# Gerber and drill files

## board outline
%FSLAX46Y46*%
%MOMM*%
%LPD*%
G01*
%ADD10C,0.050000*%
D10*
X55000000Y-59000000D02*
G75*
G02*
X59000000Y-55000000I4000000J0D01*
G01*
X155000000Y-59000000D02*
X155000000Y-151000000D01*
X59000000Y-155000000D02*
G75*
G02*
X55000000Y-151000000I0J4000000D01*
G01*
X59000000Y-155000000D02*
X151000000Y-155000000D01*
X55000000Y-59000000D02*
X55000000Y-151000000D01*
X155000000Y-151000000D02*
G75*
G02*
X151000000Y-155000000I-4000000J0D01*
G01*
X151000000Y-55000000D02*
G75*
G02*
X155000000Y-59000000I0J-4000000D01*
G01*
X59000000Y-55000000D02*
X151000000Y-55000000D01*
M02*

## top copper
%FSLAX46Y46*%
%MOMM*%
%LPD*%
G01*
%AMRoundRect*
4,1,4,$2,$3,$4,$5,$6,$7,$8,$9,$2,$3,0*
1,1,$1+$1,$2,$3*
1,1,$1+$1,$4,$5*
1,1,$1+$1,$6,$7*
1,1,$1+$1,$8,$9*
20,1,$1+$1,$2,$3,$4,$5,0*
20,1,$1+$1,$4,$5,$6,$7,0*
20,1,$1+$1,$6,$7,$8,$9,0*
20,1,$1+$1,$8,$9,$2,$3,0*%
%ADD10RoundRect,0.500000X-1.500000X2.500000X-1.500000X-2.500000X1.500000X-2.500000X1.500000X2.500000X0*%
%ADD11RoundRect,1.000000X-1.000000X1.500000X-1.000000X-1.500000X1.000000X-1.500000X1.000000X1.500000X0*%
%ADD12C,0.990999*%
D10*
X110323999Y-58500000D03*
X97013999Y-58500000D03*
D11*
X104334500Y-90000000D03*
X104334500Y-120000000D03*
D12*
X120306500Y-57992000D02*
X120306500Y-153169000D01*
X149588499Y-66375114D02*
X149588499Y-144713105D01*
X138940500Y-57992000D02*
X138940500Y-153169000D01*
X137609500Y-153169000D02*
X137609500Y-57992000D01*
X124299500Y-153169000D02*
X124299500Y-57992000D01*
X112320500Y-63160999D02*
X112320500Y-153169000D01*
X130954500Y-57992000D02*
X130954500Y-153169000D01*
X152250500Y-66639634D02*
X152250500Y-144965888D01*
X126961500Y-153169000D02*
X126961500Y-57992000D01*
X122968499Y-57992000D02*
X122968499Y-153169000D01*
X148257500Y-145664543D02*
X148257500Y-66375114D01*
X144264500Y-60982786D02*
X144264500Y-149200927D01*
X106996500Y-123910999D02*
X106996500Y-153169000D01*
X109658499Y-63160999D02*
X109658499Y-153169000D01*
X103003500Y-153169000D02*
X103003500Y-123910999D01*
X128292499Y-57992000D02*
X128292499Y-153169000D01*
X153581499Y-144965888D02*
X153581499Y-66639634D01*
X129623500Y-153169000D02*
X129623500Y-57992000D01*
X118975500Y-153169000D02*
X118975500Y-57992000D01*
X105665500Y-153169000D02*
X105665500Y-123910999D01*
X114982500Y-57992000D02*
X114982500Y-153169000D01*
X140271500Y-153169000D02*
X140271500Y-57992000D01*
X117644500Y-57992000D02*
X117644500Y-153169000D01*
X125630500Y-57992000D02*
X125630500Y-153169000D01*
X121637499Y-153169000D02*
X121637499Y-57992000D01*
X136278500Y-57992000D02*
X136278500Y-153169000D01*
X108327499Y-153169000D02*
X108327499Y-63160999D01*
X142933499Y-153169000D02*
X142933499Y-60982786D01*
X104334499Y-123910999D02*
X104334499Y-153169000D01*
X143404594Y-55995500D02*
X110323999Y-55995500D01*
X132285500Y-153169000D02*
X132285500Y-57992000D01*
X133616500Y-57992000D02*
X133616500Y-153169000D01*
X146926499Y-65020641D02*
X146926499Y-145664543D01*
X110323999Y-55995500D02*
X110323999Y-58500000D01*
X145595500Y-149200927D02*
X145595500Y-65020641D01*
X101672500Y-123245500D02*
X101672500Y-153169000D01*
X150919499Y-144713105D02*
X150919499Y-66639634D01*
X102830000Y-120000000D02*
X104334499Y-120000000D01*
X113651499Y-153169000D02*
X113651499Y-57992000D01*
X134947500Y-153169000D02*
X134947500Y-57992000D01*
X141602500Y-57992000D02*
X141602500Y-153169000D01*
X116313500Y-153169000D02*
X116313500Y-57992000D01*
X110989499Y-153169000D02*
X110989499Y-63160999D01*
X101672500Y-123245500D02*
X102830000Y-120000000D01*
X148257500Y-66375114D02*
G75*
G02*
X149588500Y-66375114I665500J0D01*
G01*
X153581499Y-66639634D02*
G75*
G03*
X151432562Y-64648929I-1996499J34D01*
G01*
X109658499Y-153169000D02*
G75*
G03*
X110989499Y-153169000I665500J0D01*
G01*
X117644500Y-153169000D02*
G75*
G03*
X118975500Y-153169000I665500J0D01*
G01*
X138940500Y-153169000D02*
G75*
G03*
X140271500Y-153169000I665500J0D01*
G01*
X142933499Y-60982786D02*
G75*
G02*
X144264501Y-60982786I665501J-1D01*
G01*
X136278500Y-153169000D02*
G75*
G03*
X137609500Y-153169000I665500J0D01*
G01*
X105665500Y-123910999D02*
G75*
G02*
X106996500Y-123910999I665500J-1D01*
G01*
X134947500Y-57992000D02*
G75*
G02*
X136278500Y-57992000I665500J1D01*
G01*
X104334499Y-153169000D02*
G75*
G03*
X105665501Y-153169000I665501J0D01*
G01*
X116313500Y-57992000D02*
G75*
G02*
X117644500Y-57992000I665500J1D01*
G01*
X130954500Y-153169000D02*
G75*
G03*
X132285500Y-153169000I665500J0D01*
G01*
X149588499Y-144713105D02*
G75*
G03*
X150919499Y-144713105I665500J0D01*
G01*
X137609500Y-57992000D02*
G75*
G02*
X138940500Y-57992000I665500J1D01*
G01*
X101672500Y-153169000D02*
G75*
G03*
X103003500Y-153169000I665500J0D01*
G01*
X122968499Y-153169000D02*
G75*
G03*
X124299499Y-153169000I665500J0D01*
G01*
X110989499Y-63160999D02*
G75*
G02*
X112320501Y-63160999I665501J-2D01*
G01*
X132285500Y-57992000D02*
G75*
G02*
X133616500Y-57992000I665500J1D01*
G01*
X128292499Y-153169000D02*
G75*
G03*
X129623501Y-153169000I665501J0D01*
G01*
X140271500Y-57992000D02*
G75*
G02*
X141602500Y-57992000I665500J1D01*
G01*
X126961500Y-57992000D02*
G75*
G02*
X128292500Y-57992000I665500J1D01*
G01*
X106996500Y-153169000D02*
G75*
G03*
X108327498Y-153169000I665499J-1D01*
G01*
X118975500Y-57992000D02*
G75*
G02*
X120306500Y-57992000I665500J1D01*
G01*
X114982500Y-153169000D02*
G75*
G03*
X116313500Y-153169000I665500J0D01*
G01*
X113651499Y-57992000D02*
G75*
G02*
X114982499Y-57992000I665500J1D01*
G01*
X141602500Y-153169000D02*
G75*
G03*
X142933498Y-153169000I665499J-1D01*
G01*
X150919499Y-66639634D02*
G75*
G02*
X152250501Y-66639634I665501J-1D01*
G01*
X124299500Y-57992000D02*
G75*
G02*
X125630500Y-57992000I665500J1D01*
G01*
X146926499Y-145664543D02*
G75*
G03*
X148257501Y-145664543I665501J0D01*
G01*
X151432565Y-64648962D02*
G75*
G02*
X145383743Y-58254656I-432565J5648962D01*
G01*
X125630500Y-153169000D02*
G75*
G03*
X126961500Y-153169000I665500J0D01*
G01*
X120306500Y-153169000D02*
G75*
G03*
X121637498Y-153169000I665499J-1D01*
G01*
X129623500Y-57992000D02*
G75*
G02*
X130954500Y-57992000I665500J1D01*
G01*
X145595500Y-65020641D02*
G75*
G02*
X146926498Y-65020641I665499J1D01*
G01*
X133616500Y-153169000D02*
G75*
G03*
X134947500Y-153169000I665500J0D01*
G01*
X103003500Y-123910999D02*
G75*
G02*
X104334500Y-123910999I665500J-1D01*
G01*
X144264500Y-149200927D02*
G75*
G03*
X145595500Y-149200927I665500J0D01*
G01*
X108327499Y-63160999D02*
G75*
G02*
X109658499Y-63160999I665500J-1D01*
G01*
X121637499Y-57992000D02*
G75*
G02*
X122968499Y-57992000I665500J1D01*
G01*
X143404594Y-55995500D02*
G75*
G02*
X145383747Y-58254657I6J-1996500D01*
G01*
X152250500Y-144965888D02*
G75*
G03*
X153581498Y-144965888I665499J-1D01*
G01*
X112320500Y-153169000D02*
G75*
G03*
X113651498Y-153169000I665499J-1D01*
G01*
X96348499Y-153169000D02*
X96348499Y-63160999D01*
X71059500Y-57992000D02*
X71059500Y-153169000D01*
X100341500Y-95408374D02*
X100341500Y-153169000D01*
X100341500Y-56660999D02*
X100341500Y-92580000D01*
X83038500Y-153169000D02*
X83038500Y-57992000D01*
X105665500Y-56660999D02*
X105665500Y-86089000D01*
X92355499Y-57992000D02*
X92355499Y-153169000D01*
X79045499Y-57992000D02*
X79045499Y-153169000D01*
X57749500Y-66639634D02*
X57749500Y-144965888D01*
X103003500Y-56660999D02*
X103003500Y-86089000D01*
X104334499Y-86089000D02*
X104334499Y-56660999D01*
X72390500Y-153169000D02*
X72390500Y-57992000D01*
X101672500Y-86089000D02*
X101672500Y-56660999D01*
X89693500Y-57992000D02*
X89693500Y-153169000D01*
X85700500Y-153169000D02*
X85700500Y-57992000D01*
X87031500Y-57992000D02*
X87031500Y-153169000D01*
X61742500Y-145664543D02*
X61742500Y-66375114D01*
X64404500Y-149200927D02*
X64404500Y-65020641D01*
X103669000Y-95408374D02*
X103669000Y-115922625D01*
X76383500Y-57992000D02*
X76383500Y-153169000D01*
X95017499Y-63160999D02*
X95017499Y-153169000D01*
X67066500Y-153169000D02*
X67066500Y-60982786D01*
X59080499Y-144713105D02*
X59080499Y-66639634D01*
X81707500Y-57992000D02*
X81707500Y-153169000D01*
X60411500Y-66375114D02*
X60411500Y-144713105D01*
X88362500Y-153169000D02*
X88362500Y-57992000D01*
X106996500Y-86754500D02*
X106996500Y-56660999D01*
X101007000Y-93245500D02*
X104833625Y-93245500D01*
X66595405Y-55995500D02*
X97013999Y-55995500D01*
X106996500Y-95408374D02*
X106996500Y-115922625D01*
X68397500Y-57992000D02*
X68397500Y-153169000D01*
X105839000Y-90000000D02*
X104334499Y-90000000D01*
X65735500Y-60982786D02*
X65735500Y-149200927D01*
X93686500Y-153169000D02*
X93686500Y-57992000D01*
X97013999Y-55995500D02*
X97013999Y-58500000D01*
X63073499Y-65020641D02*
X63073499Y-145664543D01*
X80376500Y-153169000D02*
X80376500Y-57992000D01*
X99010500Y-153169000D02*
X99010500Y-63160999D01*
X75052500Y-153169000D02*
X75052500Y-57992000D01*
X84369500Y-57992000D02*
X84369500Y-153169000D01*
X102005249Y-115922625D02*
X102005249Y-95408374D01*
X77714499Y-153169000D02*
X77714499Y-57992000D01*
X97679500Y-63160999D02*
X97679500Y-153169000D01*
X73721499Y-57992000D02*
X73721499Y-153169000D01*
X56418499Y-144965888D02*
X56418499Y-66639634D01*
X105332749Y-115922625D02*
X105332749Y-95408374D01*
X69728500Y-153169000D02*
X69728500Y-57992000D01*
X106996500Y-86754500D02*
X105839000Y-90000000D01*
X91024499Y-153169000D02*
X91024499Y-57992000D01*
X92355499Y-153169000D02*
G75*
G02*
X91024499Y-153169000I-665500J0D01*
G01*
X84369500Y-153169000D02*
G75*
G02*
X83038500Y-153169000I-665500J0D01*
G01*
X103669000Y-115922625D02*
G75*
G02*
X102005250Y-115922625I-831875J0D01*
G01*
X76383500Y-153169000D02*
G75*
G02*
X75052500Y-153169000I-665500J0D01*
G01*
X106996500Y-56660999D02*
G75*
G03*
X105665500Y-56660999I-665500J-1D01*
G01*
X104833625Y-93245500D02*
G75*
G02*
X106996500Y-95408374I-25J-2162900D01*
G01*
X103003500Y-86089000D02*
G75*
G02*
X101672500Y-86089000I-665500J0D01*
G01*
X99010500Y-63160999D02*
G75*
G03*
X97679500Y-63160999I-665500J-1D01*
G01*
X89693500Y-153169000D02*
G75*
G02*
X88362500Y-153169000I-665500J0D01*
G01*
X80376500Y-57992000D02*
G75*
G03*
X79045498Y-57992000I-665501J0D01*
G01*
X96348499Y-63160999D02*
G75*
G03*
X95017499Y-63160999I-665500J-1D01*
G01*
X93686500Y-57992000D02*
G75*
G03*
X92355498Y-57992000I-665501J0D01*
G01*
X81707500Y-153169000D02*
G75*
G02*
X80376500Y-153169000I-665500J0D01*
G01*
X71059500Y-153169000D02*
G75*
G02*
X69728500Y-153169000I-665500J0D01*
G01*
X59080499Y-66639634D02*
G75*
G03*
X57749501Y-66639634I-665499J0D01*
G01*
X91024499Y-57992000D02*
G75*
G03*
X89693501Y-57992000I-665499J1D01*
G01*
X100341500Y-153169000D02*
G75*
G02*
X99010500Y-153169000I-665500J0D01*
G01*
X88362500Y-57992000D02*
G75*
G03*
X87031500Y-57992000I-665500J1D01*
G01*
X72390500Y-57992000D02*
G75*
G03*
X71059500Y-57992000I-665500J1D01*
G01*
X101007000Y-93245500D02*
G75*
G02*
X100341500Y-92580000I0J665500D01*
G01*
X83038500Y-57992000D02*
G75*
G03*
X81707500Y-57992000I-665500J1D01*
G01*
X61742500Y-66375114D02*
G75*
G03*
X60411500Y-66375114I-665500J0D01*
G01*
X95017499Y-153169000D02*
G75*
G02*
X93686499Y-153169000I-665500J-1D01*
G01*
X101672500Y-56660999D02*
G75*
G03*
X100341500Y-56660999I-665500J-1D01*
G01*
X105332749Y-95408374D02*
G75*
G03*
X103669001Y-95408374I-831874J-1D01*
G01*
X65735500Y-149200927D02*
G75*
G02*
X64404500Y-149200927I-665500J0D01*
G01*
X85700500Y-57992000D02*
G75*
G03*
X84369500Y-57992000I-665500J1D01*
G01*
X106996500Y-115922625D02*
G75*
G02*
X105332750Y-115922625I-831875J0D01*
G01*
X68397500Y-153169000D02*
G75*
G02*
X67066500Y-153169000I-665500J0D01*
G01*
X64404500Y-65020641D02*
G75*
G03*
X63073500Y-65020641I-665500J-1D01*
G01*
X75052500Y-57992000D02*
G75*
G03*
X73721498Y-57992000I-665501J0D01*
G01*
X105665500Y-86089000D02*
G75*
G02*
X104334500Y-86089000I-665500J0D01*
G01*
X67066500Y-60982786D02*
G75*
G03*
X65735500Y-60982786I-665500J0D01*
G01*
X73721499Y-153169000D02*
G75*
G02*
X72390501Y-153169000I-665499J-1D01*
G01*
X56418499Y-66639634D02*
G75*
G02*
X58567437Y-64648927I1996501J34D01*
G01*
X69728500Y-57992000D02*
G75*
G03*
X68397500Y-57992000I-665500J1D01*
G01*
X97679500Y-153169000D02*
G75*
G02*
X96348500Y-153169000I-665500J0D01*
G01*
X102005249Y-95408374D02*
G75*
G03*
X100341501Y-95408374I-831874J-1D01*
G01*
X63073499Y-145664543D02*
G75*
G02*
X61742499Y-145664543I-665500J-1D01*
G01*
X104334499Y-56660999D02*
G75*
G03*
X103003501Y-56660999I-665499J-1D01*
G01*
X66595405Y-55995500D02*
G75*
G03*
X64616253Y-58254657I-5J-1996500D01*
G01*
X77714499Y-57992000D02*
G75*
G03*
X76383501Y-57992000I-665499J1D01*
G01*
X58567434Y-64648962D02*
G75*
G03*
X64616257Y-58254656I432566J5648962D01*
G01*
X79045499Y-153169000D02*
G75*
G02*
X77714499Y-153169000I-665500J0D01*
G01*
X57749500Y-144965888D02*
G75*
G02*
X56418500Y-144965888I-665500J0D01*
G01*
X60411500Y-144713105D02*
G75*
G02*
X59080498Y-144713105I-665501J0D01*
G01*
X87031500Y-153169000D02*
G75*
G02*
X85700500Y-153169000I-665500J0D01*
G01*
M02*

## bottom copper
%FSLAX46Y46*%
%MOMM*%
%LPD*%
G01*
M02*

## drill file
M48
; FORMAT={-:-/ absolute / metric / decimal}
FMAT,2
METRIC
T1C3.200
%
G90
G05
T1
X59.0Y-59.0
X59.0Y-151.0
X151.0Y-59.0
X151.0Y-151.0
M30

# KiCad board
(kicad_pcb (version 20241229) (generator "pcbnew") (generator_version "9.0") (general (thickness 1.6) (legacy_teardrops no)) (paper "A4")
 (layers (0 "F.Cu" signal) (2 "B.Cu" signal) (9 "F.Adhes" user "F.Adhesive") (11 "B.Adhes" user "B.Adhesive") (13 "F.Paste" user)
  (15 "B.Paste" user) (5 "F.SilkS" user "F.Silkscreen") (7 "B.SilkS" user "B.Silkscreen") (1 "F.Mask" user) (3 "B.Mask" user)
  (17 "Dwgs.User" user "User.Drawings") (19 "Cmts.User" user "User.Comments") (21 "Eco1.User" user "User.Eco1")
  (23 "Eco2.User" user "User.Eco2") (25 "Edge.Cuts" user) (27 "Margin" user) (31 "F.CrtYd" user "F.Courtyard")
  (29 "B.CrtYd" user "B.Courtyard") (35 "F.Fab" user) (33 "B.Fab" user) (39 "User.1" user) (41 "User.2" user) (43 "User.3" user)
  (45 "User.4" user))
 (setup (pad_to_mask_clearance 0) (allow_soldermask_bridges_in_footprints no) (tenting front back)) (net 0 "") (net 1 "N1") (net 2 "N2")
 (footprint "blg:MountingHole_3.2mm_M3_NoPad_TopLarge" (layer "F.Cu") (at 151 59)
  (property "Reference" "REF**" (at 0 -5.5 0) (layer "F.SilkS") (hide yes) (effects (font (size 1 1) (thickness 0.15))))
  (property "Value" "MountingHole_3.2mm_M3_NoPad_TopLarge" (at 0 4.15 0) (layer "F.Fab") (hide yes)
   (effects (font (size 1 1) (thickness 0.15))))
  (pad "" np_thru_hole circle (at 0 0) (size 7.6 7.6) (drill 3.2) (layers) (zone_connect 2)))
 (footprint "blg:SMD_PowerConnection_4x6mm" (layer "F.Cu") (at 110.323999 58.5 -90)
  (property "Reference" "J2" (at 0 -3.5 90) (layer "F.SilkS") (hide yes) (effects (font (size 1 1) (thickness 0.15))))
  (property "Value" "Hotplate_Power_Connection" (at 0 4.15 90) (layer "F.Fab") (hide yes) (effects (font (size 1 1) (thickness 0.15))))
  (pad "1" smd roundrect (at 0 0 270) (size 6 4) (layers "F.Cu" "F.Mask" "F.Paste") (roundrect_rratio 0.125) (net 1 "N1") (zone_connect 2)))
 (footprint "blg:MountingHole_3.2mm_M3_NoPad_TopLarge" (layer "F.Cu") (at 59 151)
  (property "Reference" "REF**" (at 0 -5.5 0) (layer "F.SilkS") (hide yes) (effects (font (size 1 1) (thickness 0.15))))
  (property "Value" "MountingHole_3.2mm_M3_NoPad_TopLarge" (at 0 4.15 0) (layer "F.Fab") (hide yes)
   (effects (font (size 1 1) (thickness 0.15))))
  (pad "" np_thru_hole circle (at 0 0) (size 7.6 7.6) (drill 3.2) (layers) (zone_connect 2)))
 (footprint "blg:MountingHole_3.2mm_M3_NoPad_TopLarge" (layer "F.Cu") (at 151 151)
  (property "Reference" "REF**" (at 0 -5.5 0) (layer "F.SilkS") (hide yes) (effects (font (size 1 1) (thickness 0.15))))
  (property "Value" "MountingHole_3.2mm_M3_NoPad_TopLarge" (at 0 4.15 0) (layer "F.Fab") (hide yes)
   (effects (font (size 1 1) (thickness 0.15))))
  (pad "" np_thru_hole circle (at 0 0) (size 7.6 7.6) (drill 3.2) (layers) (zone_connect 2)))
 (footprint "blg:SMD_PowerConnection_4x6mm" (layer "F.Cu") (at 97.013999 58.5 -90)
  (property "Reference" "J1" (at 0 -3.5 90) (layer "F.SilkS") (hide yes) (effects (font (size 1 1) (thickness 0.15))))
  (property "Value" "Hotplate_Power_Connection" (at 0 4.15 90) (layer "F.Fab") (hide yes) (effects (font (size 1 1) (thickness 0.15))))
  (pad "1" smd roundrect (at 0 0 270) (size 6 4) (layers "F.Cu" "F.Mask" "F.Paste") (roundrect_rratio 0.125) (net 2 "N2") (zone_connect 2)))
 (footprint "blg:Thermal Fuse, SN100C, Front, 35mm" (layer "F.Cu") (at 104.3345 105 -90)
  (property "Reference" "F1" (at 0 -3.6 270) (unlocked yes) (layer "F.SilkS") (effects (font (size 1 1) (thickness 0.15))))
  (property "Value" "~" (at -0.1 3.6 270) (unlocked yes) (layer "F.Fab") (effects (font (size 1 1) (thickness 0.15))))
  (pad "1" smd roundrect (at -15 0 270) (size 5 4) (layers "F.Cu" "F.Mask") (roundrect_rratio 0.25) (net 2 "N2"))
  (pad "2" smd roundrect (at 15 0 270) (size 5 4) (layers "F.Cu" "F.Mask") (roundrect_rratio 0.25) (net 1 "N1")))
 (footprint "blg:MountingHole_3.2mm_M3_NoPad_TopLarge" (layer "F.Cu") (at 59 59)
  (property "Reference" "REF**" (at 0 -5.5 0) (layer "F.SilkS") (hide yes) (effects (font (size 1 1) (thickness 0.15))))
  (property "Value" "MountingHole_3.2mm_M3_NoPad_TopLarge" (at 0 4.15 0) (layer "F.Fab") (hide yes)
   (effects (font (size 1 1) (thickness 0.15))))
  (pad "" np_thru_hole circle (at 0 0) (size 7.6 7.6) (drill 3.2) (layers) (zone_connect 2)))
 (gr_arc (start 55 59) (mid 56.171573 56.171573) (end 59 55) (stroke (width 0.05) (type solid)) (layer "Edge.Cuts"))
 (gr_line (start 155 59) (end 155 151) (stroke (width 0.05) (type default)) (layer "Edge.Cuts"))
 (gr_arc (start 59 155) (mid 56.171573 153.828427) (end 55 151) (stroke (width 0.05) (type solid)) (layer "Edge.Cuts"))
 (gr_line (start 59 155) (end 151 155) (stroke (width 0.05) (type default)) (layer "Edge.Cuts"))
 (gr_line (start 55 59) (end 55 151) (stroke (width 0.05) (type default)) (layer "Edge.Cuts"))
 (gr_arc (start 155 151) (mid 153.828427 153.828427) (end 151 155) (stroke (width 0.05) (type solid)) (layer "Edge.Cuts"))
 (gr_arc (start 151 55) (mid 153.828427 56.171573) (end 155 59) (stroke (width 0.05) (type solid)) (layer "Edge.Cuts"))
 (gr_line (start 59 55) (end 151 55) (stroke (width 0.05) (type default)) (layer "Edge.Cuts"))
 (segment (start 120.3065 57.992) (end 120.3065 153.169) (width 0.990999) (layer "F.Cu") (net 1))
 (segment (start 149.588499 66.375114) (end 149.588499 144.713105) (width 0.990999) (layer "F.Cu") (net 1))
 (segment (start 138.9405 57.992) (end 138.9405 153.169) (width 0.990999) (layer "F.Cu") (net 1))
 (segment (start 137.6095 153.169) (end 137.6095 57.992) (width 0.990999) (layer "F.Cu") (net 1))
 (segment (start 124.2995 153.169) (end 124.2995 57.992) (width 0.990999) (layer "F.Cu") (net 1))
 (segment (start 112.3205 63.160999) (end 112.3205 153.169) (width 0.990999) (layer "F.Cu") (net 1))
 (segment (start 130.9545 57.992) (end 130.9545 153.169) (width 0.990999) (layer "F.Cu") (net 1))
 (segment (start 152.2505 66.639634) (end 152.2505 144.965888) (width 0.990999) (layer "F.Cu") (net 1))
 (segment (start 126.9615 153.169) (end 126.9615 57.992) (width 0.990999) (layer "F.Cu") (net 1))
 (segment (start 122.968499 57.992) (end 122.968499 153.169) (width 0.990999) (layer "F.Cu") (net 1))
 (segment (start 148.2575 145.664543) (end 148.2575 66.375114) (width 0.990999) (layer "F.Cu") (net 1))
 (segment (start 144.2645 60.982786) (end 144.2645 149.200927) (width 0.990999) (layer "F.Cu") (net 1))
 (segment (start 106.9965 123.910999) (end 106.9965 153.169) (width 0.990999) (layer "F.Cu") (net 1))
 (segment (start 109.658499 63.160999) (end 109.658499 153.169) (width 0.990999) (layer "F.Cu") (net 1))
 (segment (start 103.0035 153.169) (end 103.0035 123.910999) (width 0.990999) (layer "F.Cu") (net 1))
 (segment (start 128.292499 57.992) (end 128.292499 153.169) (width 0.990999) (layer "F.Cu") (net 1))
 (segment (start 153.581499 144.965888) (end 153.581499 66.639634) (width 0.990999) (layer "F.Cu") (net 1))
 (segment (start 129.6235 153.169) (end 129.6235 57.992) (width 0.990999) (layer "F.Cu") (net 1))
 (segment (start 118.9755 153.169) (end 118.9755 57.992) (width 0.990999) (layer "F.Cu") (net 1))
 (segment (start 105.6655 153.169) (end 105.6655 123.910999) (width 0.990999) (layer "F.Cu") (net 1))
 (segment (start 114.9825 57.992) (end 114.9825 153.169) (width 0.990999) (layer "F.Cu") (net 1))
 (segment (start 140.2715 153.169) (end 140.2715 57.992) (width 0.990999) (layer "F.Cu") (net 1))
 (segment (start 117.6445 57.992) (end 117.6445 153.169) (width 0.990999) (layer "F.Cu") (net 1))
 (segment (start 125.6305 57.992) (end 125.6305 153.169) (width 0.990999) (layer "F.Cu") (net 1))
 (segment (start 121.637499 153.169) (end 121.637499 57.992) (width 0.990999) (layer "F.Cu") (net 1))
 (segment (start 136.2785 57.992) (end 136.2785 153.169) (width 0.990999) (layer "F.Cu") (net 1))
 (segment (start 108.327499 153.169) (end 108.327499 63.160999) (width 0.990999) (layer "F.Cu") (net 1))
 (segment (start 142.933499 153.169) (end 142.933499 60.982786) (width 0.990999) (layer "F.Cu") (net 1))
 (segment (start 104.334499 123.910999) (end 104.334499 153.169) (width 0.990999) (layer "F.Cu") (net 1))
 (segment (start 143.404594 55.9955) (end 110.323999 55.9955) (width 0.990999) (layer "F.Cu") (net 1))
 (segment (start 132.2855 153.169) (end 132.2855 57.992) (width 0.990999) (layer "F.Cu") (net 1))
 (segment (start 133.6165 57.992) (end 133.6165 153.169) (width 0.990999) (layer "F.Cu") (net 1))
 (segment (start 146.926499 65.020641) (end 146.926499 145.664543) (width 0.990999) (layer "F.Cu") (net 1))
 (segment (start 110.323999 55.9955) (end 110.323999 58.5) (width 0.990999) (layer "F.Cu") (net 1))
 (segment (start 145.5955 149.200927) (end 145.5955 65.020641) (width 0.990999) (layer "F.Cu") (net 1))
 (segment (start 101.6725 123.2455) (end 101.6725 153.169) (width 0.990999) (layer "F.Cu") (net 1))
 (segment (start 150.919499 144.713105) (end 150.919499 66.639634) (width 0.990999) (layer "F.Cu") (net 1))
 (segment (start 102.83 120) (end 104.334499 120) (width 0.990999) (layer "F.Cu") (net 1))
 (segment (start 113.651499 153.169) (end 113.651499 57.992) (width 0.990999) (layer "F.Cu") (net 1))
 (segment (start 134.9475 153.169) (end 134.9475 57.992) (width 0.990999) (layer "F.Cu") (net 1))
 (segment (start 141.6025 57.992) (end 141.6025 153.169) (width 0.990999) (layer "F.Cu") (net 1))
 (segment (start 116.3135 153.169) (end 116.3135 57.992) (width 0.990999) (layer "F.Cu") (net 1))
 (segment (start 110.989499 153.169) (end 110.989499 63.160999) (width 0.990999) (layer "F.Cu") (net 1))
 (segment (start 101.6725 123.2455) (end 102.83 120) (width 0.990999) (layer "F.Cu") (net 1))
 (arc (start 148.2575 66.375114) (mid 148.923 65.709614) (end 149.588499 66.375114) (width 0.990999) (layer "F.Cu") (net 1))
 (arc (start 153.581499 66.639634) (mid 153.048645 65.281785) (end 151.432565 64.648962) (width 0.990999) (layer "F.Cu") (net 1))
 (arc (start 109.658499 153.169) (mid 110.324 153.8345) (end 110.989499 153.169) (width 0.990999) (layer "F.Cu") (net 1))
 (arc (start 117.6445 153.169) (mid 118.31 153.8345) (end 118.9755 153.169) (width 0.990999) (layer "F.Cu") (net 1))
 (arc (start 138.9405 153.169) (mid 139.605999 153.8345) (end 140.2715 153.169) (width 0.990999) (layer "F.Cu") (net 1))
 (arc (start 142.933499 60.982786) (mid 143.599 60.317286) (end 144.2645 60.982786) (width 0.990999) (layer "F.Cu") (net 1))
 (arc (start 136.2785 153.169) (mid 136.944 153.8345) (end 137.6095 153.169) (width 0.990999) (layer "F.Cu") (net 1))
 (arc (start 105.6655 123.910999) (mid 106.330999 123.2455) (end 106.9965 123.910999) (width 0.990999) (layer "F.Cu") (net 1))
 (arc (start 134.9475 57.992) (mid 135.612999 57.326499) (end 136.2785 57.992) (width 0.990999) (layer "F.Cu") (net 1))
 (arc (start 104.334499 153.169) (mid 105 153.8345) (end 105.6655 153.169) (width 0.990999) (layer "F.Cu") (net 1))
 (arc (start 116.3135 57.992) (mid 116.979 57.326499) (end 117.6445 57.992) (width 0.990999) (layer "F.Cu") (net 1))
 (arc (start 130.9545 153.169) (mid 131.619999 153.8345) (end 132.2855 153.169) (width 0.990999) (layer "F.Cu") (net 1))
 (arc (start 149.588499 144.713105) (mid 150.254 145.378605) (end 150.919499 144.713105) (width 0.990999) (layer "F.Cu") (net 1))
 (arc (start 137.6095 57.992) (mid 138.274999 57.326499) (end 138.9405 57.992) (width 0.990999) (layer "F.Cu") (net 1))
 (arc (start 101.6725 153.169) (mid 102.338 153.8345) (end 103.0035 153.169) (width 0.990999) (layer "F.Cu") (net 1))
 (arc (start 122.968499 153.169) (mid 123.634 153.8345) (end 124.2995 153.169) (width 0.990999) (layer "F.Cu") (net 1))
 (arc (start 110.989499 63.160999) (mid 111.654999 62.4955) (end 112.3205 63.160999) (width 0.990999) (layer "F.Cu") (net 1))
 (arc (start 132.2855 57.992) (mid 132.951 57.326499) (end 133.6165 57.992) (width 0.990999) (layer "F.Cu") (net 1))
 (arc (start 128.292499 153.169) (mid 128.958 153.8345) (end 129.6235 153.169) (width 0.990999) (layer "F.Cu") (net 1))
 (arc (start 140.2715 57.992) (mid 140.937 57.326499) (end 141.6025 57.992) (width 0.990999) (layer "F.Cu") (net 1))
 (arc (start 126.9615 57.992) (mid 127.627 57.326499) (end 128.292499 57.992) (width 0.990999) (layer "F.Cu") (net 1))
 (arc (start 106.9965 153.169) (mid 107.661999 153.8345) (end 108.327499 153.169) (width 0.990999) (layer "F.Cu") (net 1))
 (arc (start 118.9755 57.992) (mid 119.640999 57.326499) (end 120.3065 57.992) (width 0.990999) (layer "F.Cu") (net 1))
 (arc (start 114.9825 153.169) (mid 115.648 153.8345) (end 116.3135 153.169) (width 0.990999) (layer "F.Cu") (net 1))
 (arc (start 113.651499 57.992) (mid 114.317 57.326499) (end 114.9825 57.992) (width 0.990999) (layer "F.Cu") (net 1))
 (arc (start 141.6025 153.169) (mid 142.268 153.8345) (end 142.933499 153.169) (width 0.990999) (layer "F.Cu") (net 1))
 (arc (start 150.919499 66.639634) (mid 151.585 65.974134) (end 152.2505 66.639634) (width 0.990999) (layer "F.Cu") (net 1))
 (arc (start 124.2995 57.992) (mid 124.964999 57.326499) (end 125.6305 57.992) (width 0.990999) (layer "F.Cu") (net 1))
 (arc (start 146.926499 145.664543) (mid 147.592 146.330043) (end 148.2575 145.664543) (width 0.990999) (layer "F.Cu") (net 1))
 (arc (start 151.432565 64.648962) (mid 146.884243 62.893383) (end 145.383742 58.254656) (width 0.990999) (layer "F.Cu") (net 1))
 (arc (start 125.6305 153.169) (mid 126.295999 153.8345) (end 126.9615 153.169) (width 0.990999) (layer "F.Cu") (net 1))
 (arc (start 120.3065 153.169) (mid 120.972 153.8345) (end 121.637499 153.169) (width 0.990999) (layer "F.Cu") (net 1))
 (arc (start 129.6235 57.992) (mid 130.288999 57.326499) (end 130.9545 57.992) (width 0.990999) (layer "F.Cu") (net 1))
 (arc (start 145.5955 65.020641) (mid 146.261 64.355141) (end 146.926499 65.020641) (width 0.990999) (layer "F.Cu") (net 1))
 (arc (start 133.6165 153.169) (mid 134.281999 153.8345) (end 134.9475 153.169) (width 0.990999) (layer "F.Cu") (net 1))
 (arc (start 103.0035 123.910999) (mid 103.669 123.2455) (end 104.334499 123.910999) (width 0.990999) (layer "F.Cu") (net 1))
 (arc (start 144.2645 149.200927) (mid 144.93 149.866427) (end 145.5955 149.200927) (width 0.990999) (layer "F.Cu") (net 1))
 (arc (start 108.327499 63.160999) (mid 108.993 62.4955) (end 109.658499 63.160999) (width 0.990999) (layer "F.Cu") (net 1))
 (arc (start 121.637499 57.992) (mid 122.303 57.326499) (end 122.968499 57.992) (width 0.990999) (layer "F.Cu") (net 1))
 (arc (start 143.404594 55.9955) (mid 144.906328 56.676397) (end 145.383742 58.254656) (width 0.990999) (layer "F.Cu") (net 1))
 (arc (start 152.2505 144.965888) (mid 152.916 145.631388) (end 153.581499 144.965888) (width 0.990999) (layer "F.Cu") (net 1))
 (arc (start 112.3205 153.169) (mid 112.985999 153.8345) (end 113.651499 153.169) (width 0.990999) (layer "F.Cu") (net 1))
 (segment (start 96.348499 153.169) (end 96.348499 63.160999) (width 0.990999) (layer "F.Cu") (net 2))
 (segment (start 71.0595 57.992) (end 71.0595 153.169) (width 0.990999) (layer "F.Cu") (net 2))
 (segment (start 100.3415 95.408374) (end 100.3415 153.169) (width 0.990999) (layer "F.Cu") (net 2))
 (segment (start 100.3415 56.660999) (end 100.3415 92.58) (width 0.990999) (layer "F.Cu") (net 2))
 (segment (start 83.0385 153.169) (end 83.0385 57.992) (width 0.990999) (layer "F.Cu") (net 2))
 (segment (start 105.6655 56.660999) (end 105.6655 86.089) (width 0.990999) (layer "F.Cu") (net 2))
 (segment (start 92.355499 57.992) (end 92.355499 153.169) (width 0.990999) (layer "F.Cu") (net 2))
 (segment (start 79.045499 57.992) (end 79.045499 153.169) (width 0.990999) (layer "F.Cu") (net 2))
 (segment (start 57.7495 66.639634) (end 57.7495 144.965888) (width 0.990999) (layer "F.Cu") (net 2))
 (segment (start 103.0035 56.660999) (end 103.0035 86.089) (width 0.990999) (layer "F.Cu") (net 2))
 (segment (start 104.334499 86.089) (end 104.334499 56.660999) (width 0.990999) (layer "F.Cu") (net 2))
 (segment (start 72.3905 153.169) (end 72.3905 57.992) (width 0.990999) (layer "F.Cu") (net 2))
 (segment (start 101.6725 86.089) (end 101.6725 56.660999) (width 0.990999) (layer "F.Cu") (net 2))
 (segment (start 89.6935 57.992) (end 89.6935 153.169) (width 0.990999) (layer "F.Cu") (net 2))
 (segment (start 85.7005 153.169) (end 85.7005 57.992) (width 0.990999) (layer "F.Cu") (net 2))
 (segment (start 87.0315 57.992) (end 87.0315 153.169) (width 0.990999) (layer "F.Cu") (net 2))
 (segment (start 61.7425 145.664543) (end 61.7425 66.375114) (width 0.990999) (layer "F.Cu") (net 2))
 (segment (start 64.4045 149.200927) (end 64.4045 65.020641) (width 0.990999) (layer "F.Cu") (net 2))
 (segment (start 103.669 95.408374) (end 103.669 115.922625) (width 0.990999) (layer "F.Cu") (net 2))
 (segment (start 76.3835 57.992) (end 76.3835 153.169) (width 0.990999) (layer "F.Cu") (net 2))
 (segment (start 95.017499 63.160999) (end 95.017499 153.169) (width 0.990999) (layer "F.Cu") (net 2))
 (segment (start 67.0665 153.169) (end 67.0665 60.982786) (width 0.990999) (layer "F.Cu") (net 2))
 (segment (start 59.080499 144.713105) (end 59.080499 66.639634) (width 0.990999) (layer "F.Cu") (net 2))
 (segment (start 81.7075 57.992) (end 81.7075 153.169) (width 0.990999) (layer "F.Cu") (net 2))
 (segment (start 60.4115 66.375114) (end 60.4115 144.713105) (width 0.990999) (layer "F.Cu") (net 2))
 (segment (start 88.3625 153.169) (end 88.3625 57.992) (width 0.990999) (layer "F.Cu") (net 2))
 (segment (start 106.9965 86.7545) (end 106.9965 56.660999) (width 0.990999) (layer "F.Cu") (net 2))
 (segment (start 101.007 93.2455) (end 104.833625 93.2455) (width 0.990999) (layer "F.Cu") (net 2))
 (segment (start 66.595405 55.9955) (end 97.013999 55.9955) (width 0.990999) (layer "F.Cu") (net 2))
 (segment (start 106.9965 95.408374) (end 106.9965 115.922625) (width 0.990999) (layer "F.Cu") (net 2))
 (segment (start 68.3975 57.992) (end 68.3975 153.169) (width 0.990999) (layer "F.Cu") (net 2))
 (segment (start 105.839 90) (end 104.334499 90) (width 0.990999) (layer "F.Cu") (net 2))
 (segment (start 65.7355 60.982786) (end 65.7355 149.200927) (width 0.990999) (layer "F.Cu") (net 2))
 (segment (start 93.6865 153.169) (end 93.6865 57.992) (width 0.990999) (layer "F.Cu") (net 2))
 (segment (start 97.013999 55.9955) (end 97.013999 58.5) (width 0.990999) (layer "F.Cu") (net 2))
 (segment (start 63.073499 65.020641) (end 63.073499 145.664543) (width 0.990999) (layer "F.Cu") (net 2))
 (segment (start 80.3765 153.169) (end 80.3765 57.992) (width 0.990999) (layer "F.Cu") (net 2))
 (segment (start 99.0105 153.169) (end 99.0105 63.160999) (width 0.990999) (layer "F.Cu") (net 2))
 (segment (start 75.0525 153.169) (end 75.0525 57.992) (width 0.990999) (layer "F.Cu") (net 2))
 (segment (start 84.3695 57.992) (end 84.3695 153.169) (width 0.990999) (layer "F.Cu") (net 2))
 (segment (start 102.005249 115.922625) (end 102.005249 95.408374) (width 0.990999) (layer "F.Cu") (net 2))
 (segment (start 77.714499 153.169) (end 77.714499 57.992) (width 0.990999) (layer "F.Cu") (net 2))
 (segment (start 97.6795 63.160999) (end 97.6795 153.169) (width 0.990999) (layer "F.Cu") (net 2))
 (segment (start 73.721499 57.992) (end 73.721499 153.169) (width 0.990999) (layer "F.Cu") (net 2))
 (segment (start 56.418499 144.965888) (end 56.418499 66.639634) (width 0.990999) (layer "F.Cu") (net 2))
 (segment (start 105.332749 115.922625) (end 105.332749 95.408374) (width 0.990999) (layer "F.Cu") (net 2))
 (segment (start 69.7285 153.169) (end 69.7285 57.992) (width 0.990999) (layer "F.Cu") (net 2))
 (segment (start 106.9965 86.7545) (end 105.839 90) (width 0.990999) (layer "F.Cu") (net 2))
 (segment (start 91.024499 153.169) (end 91.024499 57.992) (width 0.990999) (layer "F.Cu") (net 2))
 (arc (start 92.355499 153.169) (mid 91.69 153.8345) (end 91.024499 153.169) (width 0.990999) (layer "F.Cu") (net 2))
 (arc (start 84.3695 153.169) (mid 83.704 153.8345) (end 83.0385 153.169) (width 0.990999) (layer "F.Cu") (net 2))
 (arc (start 103.669 115.922625) (mid 102.837125 116.7545) (end 102.005249 115.922625) (width 0.990999) (layer "F.Cu") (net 2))
 (arc (start 76.3835 153.169) (mid 75.717999 153.8345) (end 75.0525 153.169) (width 0.990999) (layer "F.Cu") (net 2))
 (arc (start 106.9965 56.660999) (mid 106.330999 55.9955) (end 105.6655 56.660999) (width 0.990999) (layer "F.Cu") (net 2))
 (arc (start 104.833625 93.2455) (mid 106.363008 93.878991) (end 106.9965 95.408374) (width 0.990999) (layer "F.Cu") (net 2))
 (arc (start 103.0035 86.089) (mid 102.338 86.7545) (end 101.6725 86.089) (width 0.990999) (layer "F.Cu") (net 2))
 (arc (start 99.0105 63.160999) (mid 98.345 62.4955) (end 97.6795 63.160999) (width 0.990999) (layer "F.Cu") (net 2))
 (arc (start 89.6935 153.169) (mid 89.027999 153.8345) (end 88.3625 153.169) (width 0.990999) (layer "F.Cu") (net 2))
 (arc (start 80.3765 57.992) (mid 79.710999 57.326499) (end 79.045499 57.992) (width 0.990999) (layer "F.Cu") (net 2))
 (arc (start 96.348499 63.160999) (mid 95.683 62.4955) (end 95.017499 63.160999) (width 0.990999) (layer "F.Cu") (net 2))
 (arc (start 93.6865 57.992) (mid 93.020999 57.326499) (end 92.355499 57.992) (width 0.990999) (layer "F.Cu") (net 2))
 (arc (start 81.7075 153.169) (mid 81.042 153.8345) (end 80.3765 153.169) (width 0.990999) (layer "F.Cu") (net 2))
 (arc (start 71.0595 153.169) (mid 70.393999 153.8345) (end 69.7285 153.169) (width 0.990999) (layer "F.Cu") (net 2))
 (arc (start 59.080499 66.639634) (mid 58.414999 65.974134) (end 57.7495 66.639634) (width 0.990999) (layer "F.Cu") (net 2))
 (arc (start 91.024499 57.992) (mid 90.359 57.326499) (end 89.6935 57.992) (width 0.990999) (layer "F.Cu") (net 2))
 (arc (start 100.3415 153.169) (mid 99.676 153.8345) (end 99.0105 153.169) (width 0.990999) (layer "F.Cu") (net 2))
 (arc (start 88.3625 57.992) (mid 87.697 57.326499) (end 87.0315 57.992) (width 0.990999) (layer "F.Cu") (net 2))
 (arc (start 72.3905 57.992) (mid 71.725 57.326499) (end 71.0595 57.992) (width 0.990999) (layer "F.Cu") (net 2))
 (arc (start 101.007 93.2455) (mid 100.53642 93.050579) (end 100.3415 92.58) (width 0.990999) (layer "F.Cu") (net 2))
 (arc (start 83.0385 57.992) (mid 82.373 57.326499) (end 81.7075 57.992) (width 0.990999) (layer "F.Cu") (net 2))
 (arc (start 61.7425 66.375114) (mid 61.077 65.709614) (end 60.4115 66.375114) (width 0.990999) (layer "F.Cu") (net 2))
 (arc (start 95.017499 153.169) (mid 94.351999 153.8345) (end 93.6865 153.169) (width 0.990999) (layer "F.Cu") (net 2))
 (arc (start 101.6725 56.660999) (mid 101.007 55.9955) (end 100.3415 56.660999) (width 0.990999) (layer "F.Cu") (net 2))
 (arc (start 105.332749 95.408374) (mid 104.500875 94.5765) (end 103.669 95.408374) (width 0.990999) (layer "F.Cu") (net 2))
 (arc (start 65.7355 149.200927) (mid 65.07 149.866427) (end 64.4045 149.200927) (width 0.990999) (layer "F.Cu") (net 2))
 (arc (start 85.7005 57.992) (mid 85.035 57.326499) (end 84.3695 57.992) (width 0.990999) (layer "F.Cu") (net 2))
 (arc (start 106.9965 115.922625) (mid 106.164625 116.7545) (end 105.332749 115.922625) (width 0.990999) (layer "F.Cu") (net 2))
 (arc (start 68.3975 153.169) (mid 67.732 153.8345) (end 67.0665 153.169) (width 0.990999) (layer "F.Cu") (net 2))
 (arc (start 64.4045 65.020641) (mid 63.739 64.355141) (end 63.073499 65.020641) (width 0.990999) (layer "F.Cu") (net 2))
 (arc (start 75.0525 57.992) (mid 74.387 57.326499) (end 73.721499 57.992) (width 0.990999) (layer "F.Cu") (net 2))
 (arc (start 105.6655 86.089) (mid 105 86.7545) (end 104.334499 86.089) (width 0.990999) (layer "F.Cu") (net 2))
 (arc (start 67.0665 60.982786) (mid 66.400999 60.317286) (end 65.7355 60.982786) (width 0.990999) (layer "F.Cu") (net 2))
 (arc (start 73.721499 153.169) (mid 73.056 153.8345) (end 72.3905 153.169) (width 0.990999) (layer "F.Cu") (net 2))
 (arc (start 56.418499 66.639634) (mid 56.951354 65.281785) (end 58.567434 64.648962) (width 0.990999) (layer "F.Cu") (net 2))
 (arc (start 69.7285 57.992) (mid 69.063 57.326499) (end 68.3975 57.992) (width 0.990999) (layer "F.Cu") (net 2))
 (arc (start 97.6795 153.169) (mid 97.014 153.8345) (end 96.348499 153.169) (width 0.990999) (layer "F.Cu") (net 2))
 (arc (start 102.005249 95.408374) (mid 101.173375 94.5765) (end 100.3415 95.408374) (width 0.990999) (layer "F.Cu") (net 2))
 (arc (start 63.073499 145.664543) (mid 62.408 146.330043) (end 61.7425 145.664543) (width 0.990999) (layer "F.Cu") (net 2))
 (arc (start 104.334499 56.660999) (mid 103.669 55.9955) (end 103.0035 56.660999) (width 0.990999) (layer "F.Cu") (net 2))
 (arc (start 66.595405 55.9955) (mid 65.093671 56.676397) (end 64.616257 58.254656) (width 0.990999) (layer "F.Cu") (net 2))
 (arc (start 77.714499 57.992) (mid 77.048999 57.326499) (end 76.3835 57.992) (width 0.990999) (layer "F.Cu") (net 2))
 (arc (start 58.567434 64.648962) (mid 63.115756 62.893383) (end 64.616257 58.254656) (width 0.990999) (layer "F.Cu") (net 2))
 (arc (start 79.045499 153.169) (mid 78.38 153.8345) (end 77.714499 153.169) (width 0.990999) (layer "F.Cu") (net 2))
 (arc (start 57.7495 144.965888) (mid 57.083999 145.631388) (end 56.418499 144.965888) (width 0.990999) (layer "F.Cu") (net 2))
 (arc (start 60.4115 144.713105) (mid 59.746 145.378605) (end 59.080499 144.713105) (width 0.990999) (layer "F.Cu") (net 2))
 (arc (start 87.0315 153.169) (mid 86.366 153.8345) (end 85.7005 153.169) (width 0.990999) (layer "F.Cu") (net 2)))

